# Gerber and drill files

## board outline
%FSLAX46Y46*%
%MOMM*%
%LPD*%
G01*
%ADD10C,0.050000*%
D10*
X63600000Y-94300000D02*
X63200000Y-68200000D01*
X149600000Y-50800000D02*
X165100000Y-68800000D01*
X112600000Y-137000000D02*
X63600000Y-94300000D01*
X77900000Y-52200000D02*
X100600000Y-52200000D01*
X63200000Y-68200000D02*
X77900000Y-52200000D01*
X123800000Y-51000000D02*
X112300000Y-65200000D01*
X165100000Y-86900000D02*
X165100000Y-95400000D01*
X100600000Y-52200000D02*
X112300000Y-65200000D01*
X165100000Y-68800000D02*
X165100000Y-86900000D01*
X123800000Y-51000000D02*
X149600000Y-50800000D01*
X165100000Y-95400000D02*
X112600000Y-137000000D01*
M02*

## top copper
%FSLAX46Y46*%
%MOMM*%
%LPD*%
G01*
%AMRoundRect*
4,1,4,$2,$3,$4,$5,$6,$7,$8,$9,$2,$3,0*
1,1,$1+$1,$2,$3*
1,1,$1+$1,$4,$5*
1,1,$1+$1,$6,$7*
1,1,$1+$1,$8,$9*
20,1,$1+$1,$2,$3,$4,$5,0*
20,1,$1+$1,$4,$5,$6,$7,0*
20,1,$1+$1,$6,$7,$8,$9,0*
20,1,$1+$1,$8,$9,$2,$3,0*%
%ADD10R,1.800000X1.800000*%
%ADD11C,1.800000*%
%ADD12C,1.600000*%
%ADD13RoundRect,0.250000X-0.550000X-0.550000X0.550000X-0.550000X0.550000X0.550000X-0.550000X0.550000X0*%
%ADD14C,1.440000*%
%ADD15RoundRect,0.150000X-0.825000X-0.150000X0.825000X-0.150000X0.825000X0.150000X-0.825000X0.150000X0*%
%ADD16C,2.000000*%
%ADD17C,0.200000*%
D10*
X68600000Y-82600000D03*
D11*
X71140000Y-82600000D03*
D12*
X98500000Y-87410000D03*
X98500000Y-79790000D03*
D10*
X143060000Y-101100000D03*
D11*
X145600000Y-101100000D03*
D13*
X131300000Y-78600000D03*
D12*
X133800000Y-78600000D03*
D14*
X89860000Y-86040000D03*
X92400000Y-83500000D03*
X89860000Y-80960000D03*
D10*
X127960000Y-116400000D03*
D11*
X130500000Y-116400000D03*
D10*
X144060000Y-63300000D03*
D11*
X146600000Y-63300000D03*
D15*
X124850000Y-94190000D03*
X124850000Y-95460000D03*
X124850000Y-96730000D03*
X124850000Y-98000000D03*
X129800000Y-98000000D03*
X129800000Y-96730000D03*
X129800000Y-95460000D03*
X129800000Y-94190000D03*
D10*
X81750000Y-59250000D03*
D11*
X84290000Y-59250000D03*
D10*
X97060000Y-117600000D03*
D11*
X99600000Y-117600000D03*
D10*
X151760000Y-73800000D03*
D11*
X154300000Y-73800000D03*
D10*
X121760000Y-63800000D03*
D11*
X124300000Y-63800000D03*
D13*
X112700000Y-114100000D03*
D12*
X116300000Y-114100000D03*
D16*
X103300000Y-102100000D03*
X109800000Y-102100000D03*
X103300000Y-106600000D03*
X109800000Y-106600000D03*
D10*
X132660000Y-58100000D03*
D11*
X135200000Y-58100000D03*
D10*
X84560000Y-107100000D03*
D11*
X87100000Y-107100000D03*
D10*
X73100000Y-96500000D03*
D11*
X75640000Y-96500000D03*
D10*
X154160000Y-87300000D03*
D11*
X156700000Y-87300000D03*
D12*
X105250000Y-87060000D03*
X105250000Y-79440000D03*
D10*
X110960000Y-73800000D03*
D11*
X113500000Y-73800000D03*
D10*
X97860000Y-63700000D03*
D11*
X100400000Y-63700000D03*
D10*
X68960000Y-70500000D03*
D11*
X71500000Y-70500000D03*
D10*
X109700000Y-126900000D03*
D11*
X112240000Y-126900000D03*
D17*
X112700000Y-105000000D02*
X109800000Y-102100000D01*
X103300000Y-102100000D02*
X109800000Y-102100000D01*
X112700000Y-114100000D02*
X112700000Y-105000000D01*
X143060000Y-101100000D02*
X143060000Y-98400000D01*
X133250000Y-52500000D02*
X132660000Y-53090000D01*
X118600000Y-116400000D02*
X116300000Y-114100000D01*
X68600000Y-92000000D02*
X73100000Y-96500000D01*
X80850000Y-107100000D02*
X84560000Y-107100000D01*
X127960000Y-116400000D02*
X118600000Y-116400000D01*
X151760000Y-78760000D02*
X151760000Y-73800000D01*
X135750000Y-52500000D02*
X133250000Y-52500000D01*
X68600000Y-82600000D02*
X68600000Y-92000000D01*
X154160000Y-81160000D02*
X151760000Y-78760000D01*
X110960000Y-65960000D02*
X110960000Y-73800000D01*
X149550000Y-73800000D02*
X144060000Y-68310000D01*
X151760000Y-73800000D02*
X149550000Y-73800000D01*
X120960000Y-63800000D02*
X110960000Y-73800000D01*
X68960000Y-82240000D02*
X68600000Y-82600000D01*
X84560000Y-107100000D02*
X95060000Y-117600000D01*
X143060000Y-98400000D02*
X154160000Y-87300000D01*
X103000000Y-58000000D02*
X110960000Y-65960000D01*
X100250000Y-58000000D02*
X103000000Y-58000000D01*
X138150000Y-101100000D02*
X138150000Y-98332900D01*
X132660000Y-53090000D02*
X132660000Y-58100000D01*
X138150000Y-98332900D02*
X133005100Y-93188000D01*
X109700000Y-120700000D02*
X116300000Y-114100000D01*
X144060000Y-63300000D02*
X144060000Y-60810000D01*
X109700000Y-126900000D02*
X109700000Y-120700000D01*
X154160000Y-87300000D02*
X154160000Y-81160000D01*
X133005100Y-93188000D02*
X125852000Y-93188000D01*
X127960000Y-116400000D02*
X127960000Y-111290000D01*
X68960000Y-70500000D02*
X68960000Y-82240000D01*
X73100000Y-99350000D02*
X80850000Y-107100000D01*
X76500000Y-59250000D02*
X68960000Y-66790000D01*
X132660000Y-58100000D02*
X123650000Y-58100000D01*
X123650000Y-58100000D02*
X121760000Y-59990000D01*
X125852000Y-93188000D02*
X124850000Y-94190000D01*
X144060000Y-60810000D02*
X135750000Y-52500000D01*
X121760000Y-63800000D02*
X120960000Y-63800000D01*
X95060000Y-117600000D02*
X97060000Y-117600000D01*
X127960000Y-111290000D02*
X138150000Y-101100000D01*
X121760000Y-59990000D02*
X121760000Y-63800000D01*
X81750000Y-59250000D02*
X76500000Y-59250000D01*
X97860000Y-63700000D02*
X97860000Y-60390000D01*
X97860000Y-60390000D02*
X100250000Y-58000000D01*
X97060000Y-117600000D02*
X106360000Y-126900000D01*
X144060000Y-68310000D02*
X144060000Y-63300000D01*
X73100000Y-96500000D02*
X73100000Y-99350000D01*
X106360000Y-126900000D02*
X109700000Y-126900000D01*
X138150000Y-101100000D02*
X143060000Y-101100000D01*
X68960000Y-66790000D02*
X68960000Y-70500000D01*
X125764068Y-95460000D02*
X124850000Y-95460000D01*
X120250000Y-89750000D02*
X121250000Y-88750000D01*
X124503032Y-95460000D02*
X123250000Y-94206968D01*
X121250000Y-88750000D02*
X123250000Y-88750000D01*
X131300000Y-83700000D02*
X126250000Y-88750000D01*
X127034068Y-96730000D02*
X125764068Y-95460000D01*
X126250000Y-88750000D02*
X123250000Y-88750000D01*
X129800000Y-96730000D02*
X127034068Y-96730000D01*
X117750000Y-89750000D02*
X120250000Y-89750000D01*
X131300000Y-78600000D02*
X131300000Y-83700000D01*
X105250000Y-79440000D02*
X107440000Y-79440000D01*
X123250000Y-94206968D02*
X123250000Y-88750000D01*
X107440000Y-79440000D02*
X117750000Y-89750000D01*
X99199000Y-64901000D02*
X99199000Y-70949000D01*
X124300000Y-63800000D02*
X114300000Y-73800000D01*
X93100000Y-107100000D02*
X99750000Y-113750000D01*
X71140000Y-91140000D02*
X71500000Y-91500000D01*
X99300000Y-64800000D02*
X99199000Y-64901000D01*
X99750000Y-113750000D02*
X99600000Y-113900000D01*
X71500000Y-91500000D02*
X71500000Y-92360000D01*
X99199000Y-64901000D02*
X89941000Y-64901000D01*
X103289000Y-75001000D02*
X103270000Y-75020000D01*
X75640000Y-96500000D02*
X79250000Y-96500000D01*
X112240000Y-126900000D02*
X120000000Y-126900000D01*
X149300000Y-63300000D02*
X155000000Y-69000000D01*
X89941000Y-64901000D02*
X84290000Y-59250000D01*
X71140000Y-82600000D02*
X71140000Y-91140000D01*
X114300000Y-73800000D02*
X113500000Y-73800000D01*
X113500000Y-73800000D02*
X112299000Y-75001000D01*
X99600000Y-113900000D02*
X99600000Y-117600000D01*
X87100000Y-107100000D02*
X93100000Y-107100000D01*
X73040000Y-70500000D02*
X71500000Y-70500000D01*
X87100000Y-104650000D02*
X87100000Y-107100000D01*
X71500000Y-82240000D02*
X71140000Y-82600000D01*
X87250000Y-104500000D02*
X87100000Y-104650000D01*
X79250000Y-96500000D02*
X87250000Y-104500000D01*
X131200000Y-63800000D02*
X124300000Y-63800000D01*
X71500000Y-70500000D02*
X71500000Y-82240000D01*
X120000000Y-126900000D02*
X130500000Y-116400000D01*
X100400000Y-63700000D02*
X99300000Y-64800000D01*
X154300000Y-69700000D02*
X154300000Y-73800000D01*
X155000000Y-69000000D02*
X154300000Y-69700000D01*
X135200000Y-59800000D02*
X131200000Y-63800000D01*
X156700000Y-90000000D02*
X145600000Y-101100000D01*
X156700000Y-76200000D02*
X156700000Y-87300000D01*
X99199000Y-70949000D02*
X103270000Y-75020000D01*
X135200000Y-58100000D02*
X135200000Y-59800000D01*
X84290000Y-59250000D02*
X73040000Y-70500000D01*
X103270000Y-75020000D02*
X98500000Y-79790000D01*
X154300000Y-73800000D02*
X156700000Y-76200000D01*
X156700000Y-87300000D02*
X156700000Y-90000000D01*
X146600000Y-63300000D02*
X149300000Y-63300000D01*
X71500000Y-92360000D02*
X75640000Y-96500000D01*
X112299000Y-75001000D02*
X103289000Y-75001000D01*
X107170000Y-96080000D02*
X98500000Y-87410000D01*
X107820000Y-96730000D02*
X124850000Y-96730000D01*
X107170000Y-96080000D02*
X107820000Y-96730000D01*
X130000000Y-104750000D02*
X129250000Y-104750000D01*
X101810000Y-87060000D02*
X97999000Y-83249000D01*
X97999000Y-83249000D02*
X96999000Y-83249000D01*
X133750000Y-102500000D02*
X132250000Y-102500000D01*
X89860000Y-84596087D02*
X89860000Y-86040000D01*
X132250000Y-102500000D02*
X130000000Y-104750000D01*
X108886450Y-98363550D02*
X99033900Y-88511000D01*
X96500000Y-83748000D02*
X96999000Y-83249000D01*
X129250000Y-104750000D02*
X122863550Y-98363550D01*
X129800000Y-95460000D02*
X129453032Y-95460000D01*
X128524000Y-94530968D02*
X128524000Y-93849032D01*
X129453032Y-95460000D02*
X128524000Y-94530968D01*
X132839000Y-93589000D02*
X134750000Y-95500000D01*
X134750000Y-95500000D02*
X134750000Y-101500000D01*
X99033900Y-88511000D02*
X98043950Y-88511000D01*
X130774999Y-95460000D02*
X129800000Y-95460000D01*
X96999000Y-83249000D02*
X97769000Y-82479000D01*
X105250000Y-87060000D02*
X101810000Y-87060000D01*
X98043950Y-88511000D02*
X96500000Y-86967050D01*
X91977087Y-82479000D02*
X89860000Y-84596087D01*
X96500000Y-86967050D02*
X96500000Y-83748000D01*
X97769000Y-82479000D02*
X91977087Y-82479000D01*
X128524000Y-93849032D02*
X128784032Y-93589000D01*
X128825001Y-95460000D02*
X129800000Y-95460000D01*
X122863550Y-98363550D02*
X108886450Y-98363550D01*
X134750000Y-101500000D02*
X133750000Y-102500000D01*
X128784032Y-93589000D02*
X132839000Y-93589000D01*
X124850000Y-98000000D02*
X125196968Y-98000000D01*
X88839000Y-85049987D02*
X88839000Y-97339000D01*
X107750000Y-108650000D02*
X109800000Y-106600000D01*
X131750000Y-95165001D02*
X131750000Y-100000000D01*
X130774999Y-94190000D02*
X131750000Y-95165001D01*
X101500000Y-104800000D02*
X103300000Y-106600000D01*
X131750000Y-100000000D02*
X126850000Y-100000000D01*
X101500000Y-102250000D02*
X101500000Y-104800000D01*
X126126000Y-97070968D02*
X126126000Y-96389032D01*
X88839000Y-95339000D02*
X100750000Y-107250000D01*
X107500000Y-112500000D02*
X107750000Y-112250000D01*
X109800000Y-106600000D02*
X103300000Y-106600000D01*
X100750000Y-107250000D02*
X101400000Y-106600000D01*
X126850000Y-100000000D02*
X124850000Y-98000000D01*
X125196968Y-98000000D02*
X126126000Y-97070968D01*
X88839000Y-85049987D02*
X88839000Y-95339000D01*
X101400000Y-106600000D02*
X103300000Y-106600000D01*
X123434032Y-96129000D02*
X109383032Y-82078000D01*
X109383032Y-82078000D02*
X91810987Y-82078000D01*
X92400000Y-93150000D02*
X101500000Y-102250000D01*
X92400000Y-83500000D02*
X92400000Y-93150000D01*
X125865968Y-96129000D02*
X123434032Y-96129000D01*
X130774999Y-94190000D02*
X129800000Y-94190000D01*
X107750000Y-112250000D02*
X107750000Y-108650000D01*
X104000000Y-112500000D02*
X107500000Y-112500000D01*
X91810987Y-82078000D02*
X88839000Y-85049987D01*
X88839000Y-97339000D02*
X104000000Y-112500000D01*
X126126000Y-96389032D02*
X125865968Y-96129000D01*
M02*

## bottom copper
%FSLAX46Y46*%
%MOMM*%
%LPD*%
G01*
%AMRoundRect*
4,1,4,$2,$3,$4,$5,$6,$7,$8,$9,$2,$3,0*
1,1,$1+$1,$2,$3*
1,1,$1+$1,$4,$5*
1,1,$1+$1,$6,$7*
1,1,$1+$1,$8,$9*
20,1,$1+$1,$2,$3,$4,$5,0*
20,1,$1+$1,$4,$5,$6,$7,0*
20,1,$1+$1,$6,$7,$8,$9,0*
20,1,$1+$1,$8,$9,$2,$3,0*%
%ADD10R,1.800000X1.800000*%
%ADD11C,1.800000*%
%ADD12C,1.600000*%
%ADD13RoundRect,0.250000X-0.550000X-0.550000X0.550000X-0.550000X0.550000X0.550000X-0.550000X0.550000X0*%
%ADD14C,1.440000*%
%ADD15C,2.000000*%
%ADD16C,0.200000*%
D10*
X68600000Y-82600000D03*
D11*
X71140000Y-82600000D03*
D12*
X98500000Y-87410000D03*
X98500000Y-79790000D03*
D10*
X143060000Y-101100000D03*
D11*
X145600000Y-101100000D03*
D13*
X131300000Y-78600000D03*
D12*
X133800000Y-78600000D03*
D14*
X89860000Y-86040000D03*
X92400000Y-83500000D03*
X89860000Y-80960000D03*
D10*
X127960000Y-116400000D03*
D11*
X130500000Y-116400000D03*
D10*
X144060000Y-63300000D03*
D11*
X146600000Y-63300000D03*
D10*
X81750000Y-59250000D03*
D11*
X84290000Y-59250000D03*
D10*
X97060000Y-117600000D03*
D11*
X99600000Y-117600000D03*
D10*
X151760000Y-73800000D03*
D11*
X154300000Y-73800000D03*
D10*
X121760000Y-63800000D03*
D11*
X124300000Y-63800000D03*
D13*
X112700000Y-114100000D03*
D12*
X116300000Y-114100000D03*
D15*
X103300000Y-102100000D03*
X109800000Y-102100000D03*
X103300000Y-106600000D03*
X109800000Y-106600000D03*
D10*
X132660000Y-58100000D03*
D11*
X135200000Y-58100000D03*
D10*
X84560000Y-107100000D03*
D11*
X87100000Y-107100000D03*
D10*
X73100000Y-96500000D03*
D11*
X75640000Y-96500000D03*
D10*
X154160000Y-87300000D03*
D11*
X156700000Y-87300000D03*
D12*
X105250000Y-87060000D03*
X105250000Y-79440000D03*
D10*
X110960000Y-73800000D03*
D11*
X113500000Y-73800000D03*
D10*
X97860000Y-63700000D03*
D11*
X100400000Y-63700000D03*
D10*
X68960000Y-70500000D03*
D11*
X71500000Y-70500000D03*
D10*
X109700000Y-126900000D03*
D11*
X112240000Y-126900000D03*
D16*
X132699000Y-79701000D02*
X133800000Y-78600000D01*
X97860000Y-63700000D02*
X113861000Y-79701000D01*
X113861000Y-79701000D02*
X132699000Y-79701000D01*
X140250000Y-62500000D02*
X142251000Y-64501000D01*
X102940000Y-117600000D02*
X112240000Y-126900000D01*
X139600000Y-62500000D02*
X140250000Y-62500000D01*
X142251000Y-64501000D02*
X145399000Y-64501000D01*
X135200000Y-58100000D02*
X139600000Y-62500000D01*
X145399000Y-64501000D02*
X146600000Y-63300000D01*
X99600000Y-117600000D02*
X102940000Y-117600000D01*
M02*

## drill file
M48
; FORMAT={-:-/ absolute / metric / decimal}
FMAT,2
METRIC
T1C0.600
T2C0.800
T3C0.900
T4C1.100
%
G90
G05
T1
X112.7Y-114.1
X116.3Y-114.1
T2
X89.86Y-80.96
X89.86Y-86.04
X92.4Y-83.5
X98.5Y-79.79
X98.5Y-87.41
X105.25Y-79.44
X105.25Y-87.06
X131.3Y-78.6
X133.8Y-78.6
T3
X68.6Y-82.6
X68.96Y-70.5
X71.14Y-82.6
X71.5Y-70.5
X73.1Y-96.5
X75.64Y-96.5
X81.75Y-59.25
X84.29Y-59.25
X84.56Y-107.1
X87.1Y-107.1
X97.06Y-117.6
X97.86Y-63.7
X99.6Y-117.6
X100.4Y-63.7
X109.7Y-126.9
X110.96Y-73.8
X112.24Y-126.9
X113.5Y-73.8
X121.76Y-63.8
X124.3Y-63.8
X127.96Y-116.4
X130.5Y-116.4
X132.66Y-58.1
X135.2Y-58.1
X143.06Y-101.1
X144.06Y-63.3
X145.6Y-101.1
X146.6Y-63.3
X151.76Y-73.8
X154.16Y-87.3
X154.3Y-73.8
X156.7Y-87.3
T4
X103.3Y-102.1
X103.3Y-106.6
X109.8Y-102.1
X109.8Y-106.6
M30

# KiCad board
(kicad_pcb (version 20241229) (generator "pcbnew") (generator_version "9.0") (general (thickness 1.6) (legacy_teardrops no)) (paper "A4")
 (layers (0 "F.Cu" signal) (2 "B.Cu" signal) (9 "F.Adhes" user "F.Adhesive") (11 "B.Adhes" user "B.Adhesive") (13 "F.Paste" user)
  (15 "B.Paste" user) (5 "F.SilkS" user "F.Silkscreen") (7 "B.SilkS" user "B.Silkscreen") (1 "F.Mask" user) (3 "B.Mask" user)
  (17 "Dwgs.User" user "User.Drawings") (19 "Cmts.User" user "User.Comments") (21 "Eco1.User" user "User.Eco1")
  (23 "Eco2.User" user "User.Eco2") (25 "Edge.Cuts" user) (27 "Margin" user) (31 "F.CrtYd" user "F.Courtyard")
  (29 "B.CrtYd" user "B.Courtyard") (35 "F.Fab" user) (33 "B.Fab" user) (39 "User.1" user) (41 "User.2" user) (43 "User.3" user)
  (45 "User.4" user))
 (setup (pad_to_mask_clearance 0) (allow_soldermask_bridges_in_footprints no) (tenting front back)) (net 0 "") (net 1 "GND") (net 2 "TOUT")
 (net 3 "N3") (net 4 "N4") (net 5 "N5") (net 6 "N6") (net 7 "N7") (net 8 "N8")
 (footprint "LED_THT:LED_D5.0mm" (layer "F.Cu") (at 68.6 82.6)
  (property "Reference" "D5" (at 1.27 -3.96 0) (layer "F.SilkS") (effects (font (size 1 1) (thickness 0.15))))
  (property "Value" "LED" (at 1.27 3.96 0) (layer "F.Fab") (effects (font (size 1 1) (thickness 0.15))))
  (pad "1" thru_hole rect (at 0 0) (size 1.8 1.8) (drill 0.9) (layers "*.Cu" "*.Mask") (remove_unused_layers no) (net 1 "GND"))
  (pad "2" thru_hole circle (at 2.54 0) (size 1.8 1.8) (drill 0.9) (layers "*.Cu" "*.Mask") (remove_unused_layers no) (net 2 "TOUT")))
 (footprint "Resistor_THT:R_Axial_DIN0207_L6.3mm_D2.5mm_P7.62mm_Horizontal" (layer "F.Cu") (at 98.5 87.41 90)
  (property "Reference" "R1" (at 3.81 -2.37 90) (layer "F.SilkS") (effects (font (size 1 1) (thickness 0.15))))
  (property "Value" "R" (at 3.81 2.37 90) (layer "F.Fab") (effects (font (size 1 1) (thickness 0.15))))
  (pad "1" thru_hole circle (at 0 0 90) (size 1.6 1.6) (drill 0.8) (layers "*.Cu" "*.Mask") (remove_unused_layers no) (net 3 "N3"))
  (pad "2" thru_hole circle (at 7.62 0 90) (size 1.6 1.6) (drill 0.8) (layers "*.Cu" "*.Mask") (remove_unused_layers no) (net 2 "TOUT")))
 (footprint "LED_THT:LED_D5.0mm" (layer "F.Cu") (at 143.06 101.1)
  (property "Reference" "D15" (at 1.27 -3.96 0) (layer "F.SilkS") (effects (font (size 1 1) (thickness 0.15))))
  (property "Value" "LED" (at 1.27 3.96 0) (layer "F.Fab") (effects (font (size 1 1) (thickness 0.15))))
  (pad "1" thru_hole rect (at 0 0) (size 1.8 1.8) (drill 0.9) (layers "*.Cu" "*.Mask") (remove_unused_layers no) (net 1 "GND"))
  (pad "2" thru_hole circle (at 2.54 0) (size 1.8 1.8) (drill 0.9) (layers "*.Cu" "*.Mask") (remove_unused_layers no) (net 2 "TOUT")))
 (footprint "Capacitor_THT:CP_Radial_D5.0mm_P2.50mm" (layer "F.Cu") (at 131.3 78.6)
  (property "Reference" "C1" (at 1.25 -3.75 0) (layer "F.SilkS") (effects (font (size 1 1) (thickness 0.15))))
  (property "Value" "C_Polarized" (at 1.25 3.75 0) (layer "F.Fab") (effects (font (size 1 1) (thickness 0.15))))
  (pad "1" thru_hole roundrect (at 0 0) (size 1.6 1.6) (drill 0.8) (layers "*.Cu" "*.Mask") (remove_unused_layers no)
   (roundrect_rratio 0.15625) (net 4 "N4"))
  (pad "2" thru_hole circle (at 2.5 0) (size 1.6 1.6) (drill 0.8) (layers "*.Cu" "*.Mask") (remove_unused_layers no) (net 1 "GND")))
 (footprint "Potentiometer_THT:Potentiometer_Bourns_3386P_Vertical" (layer "F.Cu") (at 89.86 86.04)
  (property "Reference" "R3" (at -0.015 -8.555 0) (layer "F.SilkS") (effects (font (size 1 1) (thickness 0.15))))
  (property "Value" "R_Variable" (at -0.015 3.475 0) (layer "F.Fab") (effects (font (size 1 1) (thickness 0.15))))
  (pad "1" thru_hole circle (at 0 0) (size 1.44 1.44) (drill 0.8) (layers "*.Cu" "*.Mask") (remove_unused_layers no) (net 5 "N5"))
  (pad "2" thru_hole circle (at 2.54 -2.54) (size 1.44 1.44) (drill 0.8) (layers "*.Cu" "*.Mask") (remove_unused_layers no) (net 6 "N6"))
  (pad "3" thru_hole circle (at 0 -5.08) (size 1.44 1.44) (drill 0.8) (layers "*.Cu" "*.Mask") (remove_unused_layers no)))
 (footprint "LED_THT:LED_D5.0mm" (layer "F.Cu") (at 127.96 116.4)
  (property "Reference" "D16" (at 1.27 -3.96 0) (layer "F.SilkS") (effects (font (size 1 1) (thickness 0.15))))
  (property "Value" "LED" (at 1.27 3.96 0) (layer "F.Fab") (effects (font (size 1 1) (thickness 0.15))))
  (pad "1" thru_hole rect (at 0 0) (size 1.8 1.8) (drill 0.9) (layers "*.Cu" "*.Mask") (remove_unused_layers no) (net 1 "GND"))
  (pad "2" thru_hole circle (at 2.54 0) (size 1.8 1.8) (drill 0.9) (layers "*.Cu" "*.Mask") (remove_unused_layers no) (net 2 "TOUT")))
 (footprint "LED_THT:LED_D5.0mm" (layer "F.Cu") (at 144.06 63.3)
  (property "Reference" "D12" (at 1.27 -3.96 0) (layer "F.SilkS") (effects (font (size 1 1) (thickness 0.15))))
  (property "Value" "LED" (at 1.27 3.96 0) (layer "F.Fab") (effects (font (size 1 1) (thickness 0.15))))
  (pad "1" thru_hole rect (at 0 0) (size 1.8 1.8) (drill 0.9) (layers "*.Cu" "*.Mask") (remove_unused_layers no) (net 1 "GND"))
  (pad "2" thru_hole circle (at 2.54 0) (size 1.8 1.8) (drill 0.9) (layers "*.Cu" "*.Mask") (remove_unused_layers no) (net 2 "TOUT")))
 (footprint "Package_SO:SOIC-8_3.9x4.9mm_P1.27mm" (layer "F.Cu") (at 127.325 96.095)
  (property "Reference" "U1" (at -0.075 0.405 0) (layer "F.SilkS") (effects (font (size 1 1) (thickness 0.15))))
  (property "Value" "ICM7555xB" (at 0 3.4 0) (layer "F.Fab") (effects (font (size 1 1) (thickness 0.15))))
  (pad "1" smd roundrect (at -2.475 -1.905) (size 1.95 0.6) (layers "F.Cu" "F.Mask" "F.Paste") (roundrect_rratio 0.25) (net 1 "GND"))
  (pad "2" smd roundrect (at -2.475 -0.635) (size 1.95 0.6) (layers "F.Cu" "F.Mask" "F.Paste") (roundrect_rratio 0.25) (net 4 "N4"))
  (pad "3" smd roundrect (at -2.475 0.635) (size 1.95 0.6) (layers "F.Cu" "F.Mask" "F.Paste") (roundrect_rratio 0.25) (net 3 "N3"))
  (pad "4" smd roundrect (at -2.475 1.905) (size 1.95 0.6) (layers "F.Cu" "F.Mask" "F.Paste") (roundrect_rratio 0.25) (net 6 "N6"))
  (pad "5" smd roundrect (at 2.475 1.905) (size 1.95 0.6) (layers "F.Cu" "F.Mask" "F.Paste") (roundrect_rratio 0.25) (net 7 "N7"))
  (pad "6" smd roundrect (at 2.475 0.635) (size 1.95 0.6) (layers "F.Cu" "F.Mask" "F.Paste") (roundrect_rratio 0.25) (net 4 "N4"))
  (pad "7" smd roundrect (at 2.475 -0.635) (size 1.95 0.6) (layers "F.Cu" "F.Mask" "F.Paste") (roundrect_rratio 0.25) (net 5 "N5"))
  (pad "8" smd roundrect (at 2.475 -1.905) (size 1.95 0.6) (layers "F.Cu" "F.Mask" "F.Paste") (roundrect_rratio 0.25) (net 6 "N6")))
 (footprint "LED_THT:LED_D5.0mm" (layer "F.Cu") (at 81.75 59.25)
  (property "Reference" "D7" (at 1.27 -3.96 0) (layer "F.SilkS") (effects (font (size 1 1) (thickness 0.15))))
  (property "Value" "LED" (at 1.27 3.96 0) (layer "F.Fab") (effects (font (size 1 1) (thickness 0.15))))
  (pad "1" thru_hole rect (at 0 0) (size 1.8 1.8) (drill 0.9) (layers "*.Cu" "*.Mask") (remove_unused_layers no) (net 1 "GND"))
  (pad "2" thru_hole circle (at 2.54 0) (size 1.8 1.8) (drill 0.9) (layers "*.Cu" "*.Mask") (remove_unused_layers no) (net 2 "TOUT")))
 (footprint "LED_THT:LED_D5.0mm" (layer "F.Cu") (at 97.06 117.6)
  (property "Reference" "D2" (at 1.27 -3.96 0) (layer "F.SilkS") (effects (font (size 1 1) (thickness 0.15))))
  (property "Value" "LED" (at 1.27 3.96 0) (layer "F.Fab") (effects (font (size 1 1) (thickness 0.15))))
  (pad "1" thru_hole rect (at 0 0) (size 1.8 1.8) (drill 0.9) (layers "*.Cu" "*.Mask") (remove_unused_layers no) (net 1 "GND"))
  (pad "2" thru_hole circle (at 2.54 0) (size 1.8 1.8) (drill 0.9) (layers "*.Cu" "*.Mask") (remove_unused_layers no) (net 2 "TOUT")))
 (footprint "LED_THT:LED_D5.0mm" (layer "F.Cu") (at 151.76 73.8)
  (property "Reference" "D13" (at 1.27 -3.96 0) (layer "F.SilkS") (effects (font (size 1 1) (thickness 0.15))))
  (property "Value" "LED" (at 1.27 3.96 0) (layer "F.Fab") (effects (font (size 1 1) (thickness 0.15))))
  (pad "1" thru_hole rect (at 0 0) (size 1.8 1.8) (drill 0.9) (layers "*.Cu" "*.Mask") (remove_unused_layers no) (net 1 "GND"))
  (pad "2" thru_hole circle (at 2.54 0) (size 1.8 1.8) (drill 0.9) (layers "*.Cu" "*.Mask") (remove_unused_layers no) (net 2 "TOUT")))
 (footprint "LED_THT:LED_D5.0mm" (layer "F.Cu") (at 121.76 63.8)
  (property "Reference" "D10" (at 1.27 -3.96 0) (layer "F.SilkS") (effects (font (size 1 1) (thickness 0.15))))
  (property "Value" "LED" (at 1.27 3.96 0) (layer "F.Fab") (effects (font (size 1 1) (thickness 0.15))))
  (pad "1" thru_hole rect (at 0 0) (size 1.8 1.8) (drill 0.9) (layers "*.Cu" "*.Mask") (remove_unused_layers no) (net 1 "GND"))
  (pad "2" thru_hole circle (at 2.54 0) (size 1.8 1.8) (drill 0.9) (layers "*.Cu" "*.Mask") (remove_unused_layers no) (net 2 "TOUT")))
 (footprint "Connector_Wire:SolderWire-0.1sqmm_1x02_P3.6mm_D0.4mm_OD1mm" (layer "F.Cu") (at 112.7 114.1)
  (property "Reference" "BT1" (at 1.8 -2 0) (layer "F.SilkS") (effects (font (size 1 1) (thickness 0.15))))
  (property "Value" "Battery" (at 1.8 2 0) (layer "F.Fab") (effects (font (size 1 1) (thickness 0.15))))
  (pad "1" thru_hole roundrect (at 0 0) (size 1.6 1.6) (drill 0.6) (layers "*.Cu" "*.Mask") (remove_unused_layers no)
   (roundrect_rratio 0.15625) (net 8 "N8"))
  (pad "2" thru_hole circle (at 3.6 0) (size 1.6 1.6) (drill 0.6) (layers "*.Cu" "*.Mask") (remove_unused_layers no) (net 1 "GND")))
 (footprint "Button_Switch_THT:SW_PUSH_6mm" (layer "F.Cu") (at 103.3 102.1)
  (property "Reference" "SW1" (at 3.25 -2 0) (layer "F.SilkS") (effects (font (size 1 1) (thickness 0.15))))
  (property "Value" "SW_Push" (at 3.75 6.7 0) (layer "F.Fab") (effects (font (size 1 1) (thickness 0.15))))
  (pad "1" thru_hole circle (at 0 0 90) (size 2 2) (drill 1.1) (layers "*.Cu" "*.Mask") (remove_unused_layers no) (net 8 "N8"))
  (pad "1" thru_hole circle (at 6.5 0 90) (size 2 2) (drill 1.1) (layers "*.Cu" "*.Mask") (remove_unused_layers no) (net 8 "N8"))
  (pad "2" thru_hole circle (at 0 4.5 90) (size 2 2) (drill 1.1) (layers "*.Cu" "*.Mask") (remove_unused_layers no) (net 6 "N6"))
  (pad "2" thru_hole circle (at 6.5 4.5 90) (size 2 2) (drill 1.1) (layers "*.Cu" "*.Mask") (remove_unused_layers no) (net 6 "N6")))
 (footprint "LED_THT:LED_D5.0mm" (layer "F.Cu") (at 132.66 58.1)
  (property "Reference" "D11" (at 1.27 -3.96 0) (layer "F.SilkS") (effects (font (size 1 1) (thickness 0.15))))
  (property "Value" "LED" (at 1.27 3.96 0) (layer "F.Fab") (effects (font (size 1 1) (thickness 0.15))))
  (pad "1" thru_hole rect (at 0 0) (size 1.8 1.8) (drill 0.9) (layers "*.Cu" "*.Mask") (remove_unused_layers no) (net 1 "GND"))
  (pad "2" thru_hole circle (at 2.54 0) (size 1.8 1.8) (drill 0.9) (layers "*.Cu" "*.Mask") (remove_unused_layers no) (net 2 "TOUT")))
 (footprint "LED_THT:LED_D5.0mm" (layer "F.Cu") (at 84.56 107.1)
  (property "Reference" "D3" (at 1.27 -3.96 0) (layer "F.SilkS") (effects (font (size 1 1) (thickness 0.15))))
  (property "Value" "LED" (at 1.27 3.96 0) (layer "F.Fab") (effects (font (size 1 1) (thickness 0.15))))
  (pad "1" thru_hole rect (at 0 0) (size 1.8 1.8) (drill 0.9) (layers "*.Cu" "*.Mask") (remove_unused_layers no) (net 1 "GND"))
  (pad "2" thru_hole circle (at 2.54 0) (size 1.8 1.8) (drill 0.9) (layers "*.Cu" "*.Mask") (remove_unused_layers no) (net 2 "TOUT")))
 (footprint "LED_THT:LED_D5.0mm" (layer "F.Cu") (at 73.1 96.5)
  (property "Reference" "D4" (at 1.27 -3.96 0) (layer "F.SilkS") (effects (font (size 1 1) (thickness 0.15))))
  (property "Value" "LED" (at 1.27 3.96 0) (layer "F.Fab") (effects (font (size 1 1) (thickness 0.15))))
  (pad "1" thru_hole rect (at 0 0) (size 1.8 1.8) (drill 0.9) (layers "*.Cu" "*.Mask") (remove_unused_layers no) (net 1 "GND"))
  (pad "2" thru_hole circle (at 2.54 0) (size 1.8 1.8) (drill 0.9) (layers "*.Cu" "*.Mask") (remove_unused_layers no) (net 2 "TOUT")))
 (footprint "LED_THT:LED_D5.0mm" (layer "F.Cu") (at 154.16 87.3)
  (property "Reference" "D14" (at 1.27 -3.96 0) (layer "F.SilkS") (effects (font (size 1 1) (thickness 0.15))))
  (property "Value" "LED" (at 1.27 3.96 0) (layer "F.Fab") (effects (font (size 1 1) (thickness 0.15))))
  (pad "1" thru_hole rect (at 0 0) (size 1.8 1.8) (drill 0.9) (layers "*.Cu" "*.Mask") (remove_unused_layers no) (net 1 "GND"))
  (pad "2" thru_hole circle (at 2.54 0) (size 1.8 1.8) (drill 0.9) (layers "*.Cu" "*.Mask") (remove_unused_layers no) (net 2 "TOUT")))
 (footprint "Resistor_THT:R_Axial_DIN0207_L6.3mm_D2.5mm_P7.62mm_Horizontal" (layer "F.Cu") (at 105.25 87.06 90)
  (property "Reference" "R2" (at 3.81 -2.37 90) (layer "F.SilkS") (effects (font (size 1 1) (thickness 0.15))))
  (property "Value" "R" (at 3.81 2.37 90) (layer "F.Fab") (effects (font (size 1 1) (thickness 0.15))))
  (pad "1" thru_hole circle (at 0 0 90) (size 1.6 1.6) (drill 0.8) (layers "*.Cu" "*.Mask") (remove_unused_layers no) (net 5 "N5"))
  (pad "2" thru_hole circle (at 7.62 0 90) (size 1.6 1.6) (drill 0.8) (layers "*.Cu" "*.Mask") (remove_unused_layers no) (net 4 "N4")))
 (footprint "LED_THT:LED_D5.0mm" (layer "F.Cu") (at 110.96 73.8)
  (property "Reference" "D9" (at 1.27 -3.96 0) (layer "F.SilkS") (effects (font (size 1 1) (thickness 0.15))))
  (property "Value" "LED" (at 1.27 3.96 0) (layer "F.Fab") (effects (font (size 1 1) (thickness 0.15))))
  (pad "1" thru_hole rect (at 0 0) (size 1.8 1.8) (drill 0.9) (layers "*.Cu" "*.Mask") (remove_unused_layers no) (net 1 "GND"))
  (pad "2" thru_hole circle (at 2.54 0) (size 1.8 1.8) (drill 0.9) (layers "*.Cu" "*.Mask") (remove_unused_layers no) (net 2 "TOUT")))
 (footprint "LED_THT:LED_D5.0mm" (layer "F.Cu") (at 97.86 63.7)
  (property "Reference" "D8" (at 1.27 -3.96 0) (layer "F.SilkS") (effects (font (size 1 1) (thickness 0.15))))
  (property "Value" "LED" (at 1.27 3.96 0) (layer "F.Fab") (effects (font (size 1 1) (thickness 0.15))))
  (pad "1" thru_hole rect (at 0 0) (size 1.8 1.8) (drill 0.9) (layers "*.Cu" "*.Mask") (remove_unused_layers no) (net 1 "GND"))
  (pad "2" thru_hole circle (at 2.54 0) (size 1.8 1.8) (drill 0.9) (layers "*.Cu" "*.Mask") (remove_unused_layers no) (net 2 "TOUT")))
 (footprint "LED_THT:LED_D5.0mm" (layer "F.Cu") (at 68.96 70.5)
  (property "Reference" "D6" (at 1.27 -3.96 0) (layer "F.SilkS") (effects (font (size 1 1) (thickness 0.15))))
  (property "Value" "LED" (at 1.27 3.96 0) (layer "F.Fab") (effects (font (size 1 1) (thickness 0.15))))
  (pad "1" thru_hole rect (at 0 0) (size 1.8 1.8) (drill 0.9) (layers "*.Cu" "*.Mask") (remove_unused_layers no) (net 1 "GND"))
  (pad "2" thru_hole circle (at 2.54 0) (size 1.8 1.8) (drill 0.9) (layers "*.Cu" "*.Mask") (remove_unused_layers no) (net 2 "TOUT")))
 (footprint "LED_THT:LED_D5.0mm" (layer "F.Cu") (at 109.7 126.9)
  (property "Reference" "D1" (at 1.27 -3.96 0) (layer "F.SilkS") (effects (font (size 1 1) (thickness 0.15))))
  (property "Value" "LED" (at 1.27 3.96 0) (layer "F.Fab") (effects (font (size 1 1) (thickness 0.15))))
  (pad "1" thru_hole rect (at 0 0) (size 1.8 1.8) (drill 0.9) (layers "*.Cu" "*.Mask") (remove_unused_layers no) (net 1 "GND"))
  (pad "2" thru_hole circle (at 2.54 0) (size 1.8 1.8) (drill 0.9) (layers "*.Cu" "*.Mask") (remove_unused_layers no) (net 2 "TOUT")))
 (gr_line (start 63.6 94.3) (end 63.2 68.2) (stroke (width 0.05) (type default)) (layer "Edge.Cuts"))
 (gr_line (start 149.6 50.8) (end 165.1 68.8) (stroke (width 0.05) (type default)) (layer "Edge.Cuts"))
 (gr_line (start 112.6 137) (end 63.6 94.3) (stroke (width 0.05) (type default)) (layer "Edge.Cuts"))
 (gr_line (start 77.9 52.2) (end 100.6 52.2) (stroke (width 0.05) (type default)) (layer "Edge.Cuts"))
 (gr_line (start 63.2 68.2) (end 77.9 52.2) (stroke (width 0.05) (type default)) (layer "Edge.Cuts"))
 (gr_line (start 123.8 51) (end 112.3 65.2) (stroke (width 0.05) (type default)) (layer "Edge.Cuts"))
 (gr_line (start 165.1 86.9) (end 165.1 95.4) (stroke (width 0.05) (type default)) (layer "Edge.Cuts"))
 (gr_line (start 100.6 52.2) (end 112.3 65.2) (stroke (width 0.05) (type default)) (layer "Edge.Cuts"))
 (gr_line (start 165.1 68.8) (end 165.1 86.9) (stroke (width 0.05) (type default)) (layer "Edge.Cuts"))
 (gr_line (start 123.8 51) (end 149.6 50.8) (stroke (width 0.05) (type default)) (layer "Edge.Cuts"))
 (gr_line (start 165.1 95.4) (end 112.6 137) (stroke (width 0.05) (type default)) (layer "Edge.Cuts"))
 (segment (start 112.7 105) (end 109.8 102.1) (width 0.2) (layer "F.Cu") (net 8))
 (segment (start 103.3 102.1) (end 109.8 102.1) (width 0.2) (layer "F.Cu") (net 8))
 (segment (start 112.7 114.1) (end 112.7 105) (width 0.2) (layer "F.Cu") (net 8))
 (segment (start 143.06 101.1) (end 143.06 98.4) (width 0.2) (layer "F.Cu") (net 1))
 (segment (start 133.25 52.5) (end 132.66 53.09) (width 0.2) (layer "F.Cu") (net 1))
 (segment (start 118.6 116.4) (end 116.3 114.1) (width 0.2) (layer "F.Cu") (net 1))
 (segment (start 68.6 92) (end 73.1 96.5) (width 0.2) (layer "F.Cu") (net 1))
 (segment (start 80.85 107.1) (end 84.56 107.1) (width 0.2) (layer "F.Cu") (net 1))
 (segment (start 127.96 116.4) (end 118.6 116.4) (width 0.2) (layer "F.Cu") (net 1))
 (segment (start 151.76 78.76) (end 151.76 73.8) (width 0.2) (layer "F.Cu") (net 1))
 (segment (start 135.75 52.5) (end 133.25 52.5) (width 0.2) (layer "F.Cu") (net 1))
 (segment (start 68.6 82.6) (end 68.6 92) (width 0.2) (layer "F.Cu") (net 1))
 (segment (start 154.16 81.16) (end 151.76 78.76) (width 0.2) (layer "F.Cu") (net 1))
 (segment (start 110.96 65.96) (end 110.96 73.8) (width 0.2) (layer "F.Cu") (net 1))
 (segment (start 149.55 73.8) (end 144.06 68.31) (width 0.2) (layer "F.Cu") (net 1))
 (segment (start 151.76 73.8) (end 149.55 73.8) (width 0.2) (layer "F.Cu") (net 1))
 (segment (start 120.96 63.8) (end 110.96 73.8) (width 0.2) (layer "F.Cu") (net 1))
 (segment (start 68.96 82.24) (end 68.6 82.6) (width 0.2) (layer "F.Cu") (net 1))
 (segment (start 84.56 107.1) (end 95.06 117.6) (width 0.2) (layer "F.Cu") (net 1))
 (segment (start 143.06 98.4) (end 154.16 87.3) (width 0.2) (layer "F.Cu") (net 1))
 (segment (start 103 58) (end 110.96 65.96) (width 0.2) (layer "F.Cu") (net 1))
 (segment (start 100.25 58) (end 103 58) (width 0.2) (layer "F.Cu") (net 1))
 (segment (start 138.15 101.1) (end 138.15 98.3329) (width 0.2) (layer "F.Cu") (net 1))
 (segment (start 132.66 53.09) (end 132.66 58.1) (width 0.2) (layer "F.Cu") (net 1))
 (segment (start 138.15 98.3329) (end 133.0051 93.188) (width 0.2) (layer "F.Cu") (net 1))
 (segment (start 109.7 120.7) (end 116.3 114.1) (width 0.2) (layer "F.Cu") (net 1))
 (segment (start 144.06 63.3) (end 144.06 60.81) (width 0.2) (layer "F.Cu") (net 1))
 (segment (start 109.7 126.9) (end 109.7 120.7) (width 0.2) (layer "F.Cu") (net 1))
 (segment (start 154.16 87.3) (end 154.16 81.16) (width 0.2) (layer "F.Cu") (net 1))
 (segment (start 133.0051 93.188) (end 125.852 93.188) (width 0.2) (layer "F.Cu") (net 1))
 (segment (start 127.96 116.4) (end 127.96 111.29) (width 0.2) (layer "F.Cu") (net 1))
 (segment (start 68.96 70.5) (end 68.96 82.24) (width 0.2) (layer "F.Cu") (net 1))
 (segment (start 73.1 99.35) (end 80.85 107.1) (width 0.2) (layer "F.Cu") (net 1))
 (segment (start 76.5 59.25) (end 68.96 66.79) (width 0.2) (layer "F.Cu") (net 1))
 (segment (start 132.66 58.1) (end 123.65 58.1) (width 0.2) (layer "F.Cu") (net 1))
 (segment (start 123.65 58.1) (end 121.76 59.99) (width 0.2) (layer "F.Cu") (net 1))
 (segment (start 125.852 93.188) (end 124.85 94.19) (width 0.2) (layer "F.Cu") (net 1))
 (segment (start 144.06 60.81) (end 135.75 52.5) (width 0.2) (layer "F.Cu") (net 1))
 (segment (start 121.76 63.8) (end 120.96 63.8) (width 0.2) (layer "F.Cu") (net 1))
 (segment (start 95.06 117.6) (end 97.06 117.6) (width 0.2) (layer "F.Cu") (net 1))
 (segment (start 127.96 111.29) (end 138.15 101.1) (width 0.2) (layer "F.Cu") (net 1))
 (segment (start 121.76 59.99) (end 121.76 63.8) (width 0.2) (layer "F.Cu") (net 1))
 (segment (start 81.75 59.25) (end 76.5 59.25) (width 0.2) (layer "F.Cu") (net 1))
 (segment (start 97.86 63.7) (end 97.86 60.39) (width 0.2) (layer "F.Cu") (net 1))
 (segment (start 97.86 60.39) (end 100.25 58) (width 0.2) (layer "F.Cu") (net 1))
 (segment (start 97.06 117.6) (end 106.36 126.9) (width 0.2) (layer "F.Cu") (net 1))
 (segment (start 144.06 68.31) (end 144.06 63.3) (width 0.2) (layer "F.Cu") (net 1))
 (segment (start 73.1 96.5) (end 73.1 99.35) (width 0.2) (layer "F.Cu") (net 1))
 (segment (start 106.36 126.9) (end 109.7 126.9) (width 0.2) (layer "F.Cu") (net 1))
 (segment (start 138.15 101.1) (end 143.06 101.1) (width 0.2) (layer "F.Cu") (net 1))
 (segment (start 68.96 66.79) (end 68.96 70.5) (width 0.2) (layer "F.Cu") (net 1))
 (segment (start 132.699 79.701) (end 133.8 78.6) (width 0.2) (layer "B.Cu") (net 1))
 (segment (start 97.86 63.7) (end 113.861 79.701) (width 0.2) (layer "B.Cu") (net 1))
 (segment (start 113.861 79.701) (end 132.699 79.701) (width 0.2) (layer "B.Cu") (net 1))
 (segment (start 125.764068 95.46) (end 124.85 95.46) (width 0.2) (layer "F.Cu") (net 4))
 (segment (start 120.25 89.75) (end 121.25 88.75) (width 0.2) (layer "F.Cu") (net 4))
 (segment (start 124.503032 95.46) (end 123.25 94.206968) (width 0.2) (layer "F.Cu") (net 4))
 (segment (start 121.25 88.75) (end 123.25 88.75) (width 0.2) (layer "F.Cu") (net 4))
 (segment (start 131.3 83.7) (end 126.25 88.75) (width 0.2) (layer "F.Cu") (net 4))
 (segment (start 127.034068 96.73) (end 125.764068 95.46) (width 0.2) (layer "F.Cu") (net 4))
 (segment (start 126.25 88.75) (end 123.25 88.75) (width 0.2) (layer "F.Cu") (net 4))
 (segment (start 129.8 96.73) (end 127.034068 96.73) (width 0.2) (layer "F.Cu") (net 4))
 (segment (start 117.75 89.75) (end 120.25 89.75) (width 0.2) (layer "F.Cu") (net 4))
 (segment (start 131.3 78.6) (end 131.3 83.7) (width 0.2) (layer "F.Cu") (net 4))
 (segment (start 105.25 79.44) (end 107.44 79.44) (width 0.2) (layer "F.Cu") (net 4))
 (segment (start 123.25 94.206968) (end 123.25 88.75) (width 0.2) (layer "F.Cu") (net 4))
 (segment (start 107.44 79.44) (end 117.75 89.75) (width 0.2) (layer "F.Cu") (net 4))
 (segment (start 99.199 64.901) (end 99.199 70.949) (width 0.2) (layer "F.Cu") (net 2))
 (segment (start 124.3 63.8) (end 114.3 73.8) (width 0.2) (layer "F.Cu") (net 2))
 (segment (start 93.1 107.1) (end 99.75 113.75) (width 0.2) (layer "F.Cu") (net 2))
 (segment (start 71.14 91.14) (end 71.5 91.5) (width 0.2) (layer "F.Cu") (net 2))
 (segment (start 99.3 64.8) (end 99.199 64.901) (width 0.2) (layer "F.Cu") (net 2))
 (segment (start 99.75 113.75) (end 99.6 113.9) (width 0.2) (layer "F.Cu") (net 2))
 (segment (start 71.5 91.5) (end 71.5 92.36) (width 0.2) (layer "F.Cu") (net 2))
 (segment (start 99.199 64.901) (end 89.941 64.901) (width 0.2) (layer "F.Cu") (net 2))
 (segment (start 103.289 75.001) (end 103.27 75.02) (width 0.2) (layer "F.Cu") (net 2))
 (segment (start 75.64 96.5) (end 79.25 96.5) (width 0.2) (layer "F.Cu") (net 2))
 (segment (start 112.24 126.9) (end 120 126.9) (width 0.2) (layer "F.Cu") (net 2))
 (segment (start 149.3 63.3) (end 155 69) (width 0.2) (layer "F.Cu") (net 2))
 (segment (start 89.941 64.901) (end 84.29 59.25) (width 0.2) (layer "F.Cu") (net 2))
 (segment (start 71.14 82.6) (end 71.14 91.14) (width 0.2) (layer "F.Cu") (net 2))
 (segment (start 114.3 73.8) (end 113.5 73.8) (width 0.2) (layer "F.Cu") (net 2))
 (segment (start 113.5 73.8) (end 112.299 75.001) (width 0.2) (layer "F.Cu") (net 2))
 (segment (start 99.6 113.9) (end 99.6 117.6) (width 0.2) (layer "F.Cu") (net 2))
 (segment (start 87.1 107.1) (end 93.1 107.1) (width 0.2) (layer "F.Cu") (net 2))
 (segment (start 73.04 70.5) (end 71.5 70.5) (width 0.2) (layer "F.Cu") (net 2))
 (segment (start 87.1 104.65) (end 87.1 107.1) (width 0.2) (layer "F.Cu") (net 2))
 (segment (start 71.5 82.24) (end 71.14 82.6) (width 0.2) (layer "F.Cu") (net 2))
 (segment (start 87.25 104.5) (end 87.1 104.65) (width 0.2) (layer "F.Cu") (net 2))
 (segment (start 79.25 96.5) (end 87.25 104.5) (width 0.2) (layer "F.Cu") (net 2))
 (segment (start 131.2 63.8) (end 124.3 63.8) (width 0.2) (layer "F.Cu") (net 2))
 (segment (start 71.5 70.5) (end 71.5 82.24) (width 0.2) (layer "F.Cu") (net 2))
 (segment (start 120 126.9) (end 130.5 116.4) (width 0.2) (layer "F.Cu") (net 2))
 (segment (start 100.4 63.7) (end 99.3 64.8) (width 0.2) (layer "F.Cu") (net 2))
 (segment (start 154.3 69.7) (end 154.3 73.8) (width 0.2) (layer "F.Cu") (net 2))
 (segment (start 155 69) (end 154.3 69.7) (width 0.2) (layer "F.Cu") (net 2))
 (segment (start 135.2 59.8) (end 131.2 63.8) (width 0.2) (layer "F.Cu") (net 2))
 (segment (start 156.7 90) (end 145.6 101.1) (width 0.2) (layer "F.Cu") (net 2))
 (segment (start 156.7 76.2) (end 156.7 87.3) (width 0.2) (layer "F.Cu") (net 2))
 (segment (start 99.199 70.949) (end 103.27 75.02) (width 0.2) (layer "F.Cu") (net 2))
 (segment (start 135.2 58.1) (end 135.2 59.8) (width 0.2) (layer "F.Cu") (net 2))
 (segment (start 84.29 59.25) (end 73.04 70.5) (width 0.2) (layer "F.Cu") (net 2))
 (segment (start 103.27 75.02) (end 98.5 79.79) (width 0.2) (layer "F.Cu") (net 2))
 (segment (start 154.3 73.8) (end 156.7 76.2) (width 0.2) (layer "F.Cu") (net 2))
 (segment (start 156.7 87.3) (end 156.7 90) (width 0.2) (layer "F.Cu") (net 2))
 (segment (start 146.6 63.3) (end 149.3 63.3) (width 0.2) (layer "F.Cu") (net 2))
 (segment (start 71.5 92.36) (end 75.64 96.5) (width 0.2) (layer "F.Cu") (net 2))
 (segment (start 112.299 75.001) (end 103.289 75.001) (width 0.2) (layer "F.Cu") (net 2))
 (segment (start 140.25 62.5) (end 142.251 64.501) (width 0.2) (layer "B.Cu") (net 2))
 (segment (start 102.94 117.6) (end 112.24 126.9) (width 0.2) (layer "B.Cu") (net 2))
 (segment (start 139.6 62.5) (end 140.25 62.5) (width 0.2) (layer "B.Cu") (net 2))
 (segment (start 142.251 64.501) (end 145.399 64.501) (width 0.2) (layer "B.Cu") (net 2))
 (segment (start 135.2 58.1) (end 139.6 62.5) (width 0.2) (layer "B.Cu") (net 2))
 (segment (start 145.399 64.501) (end 146.6 63.3) (width 0.2) (layer "B.Cu") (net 2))
 (segment (start 99.6 117.6) (end 102.94 117.6) (width 0.2) (layer "B.Cu") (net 2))
 (segment (start 107.17 96.08) (end 98.5 87.41) (width 0.2) (layer "F.Cu") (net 3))
 (segment (start 107.82 96.73) (end 124.85 96.73) (width 0.2) (layer "F.Cu") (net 3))
 (segment (start 107.17 96.08) (end 107.82 96.73) (width 0.2) (layer "F.Cu") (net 3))
 (segment (start 130 104.75) (end 129.25 104.75) (width 0.2) (layer "F.Cu") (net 5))
 (segment (start 101.81 87.06) (end 97.999 83.249) (width 0.2) (layer "F.Cu") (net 5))
 (segment (start 97.999 83.249) (end 96.999 83.249) (width 0.2) (layer "F.Cu") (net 5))
 (segment (start 133.75 102.5) (end 132.25 102.5) (width 0.2) (layer "F.Cu") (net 5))
 (segment (start 89.86 84.596087) (end 89.86 86.04) (width 0.2) (layer "F.Cu") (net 5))
 (segment (start 132.25 102.5) (end 130 104.75) (width 0.2) (layer "F.Cu") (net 5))
 (segment (start 108.88645 98.36355) (end 99.0339 88.511) (width 0.2) (layer "F.Cu") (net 5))
 (segment (start 96.5 83.748) (end 96.999 83.249) (width 0.2) (layer "F.Cu") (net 5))
 (segment (start 129.25 104.75) (end 122.86355 98.36355) (width 0.2) (layer "F.Cu") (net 5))
 (segment (start 129.8 95.46) (end 129.453032 95.46) (width 0.2) (layer "F.Cu") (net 5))
 (segment (start 128.524 94.530968) (end 128.524 93.849032) (width 0.2) (layer "F.Cu") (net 5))
 (segment (start 129.453032 95.46) (end 128.524 94.530968) (width 0.2) (layer "F.Cu") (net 5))
 (segment (start 132.839 93.589) (end 134.75 95.5) (width 0.2) (layer "F.Cu") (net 5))
 (segment (start 134.75 95.5) (end 134.75 101.5) (width 0.2) (layer "F.Cu") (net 5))
 (segment (start 99.0339 88.511) (end 98.04395 88.511) (width 0.2) (layer "F.Cu") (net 5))
 (segment (start 130.774999 95.46) (end 129.8 95.46) (width 0.2) (layer "F.Cu") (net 5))
 (segment (start 96.999 83.249) (end 97.769 82.479) (width 0.2) (layer "F.Cu") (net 5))
 (segment (start 105.25 87.06) (end 101.81 87.06) (width 0.2) (layer "F.Cu") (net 5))
 (segment (start 98.04395 88.511) (end 96.5 86.96705) (width 0.2) (layer "F.Cu") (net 5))
 (segment (start 91.977087 82.479) (end 89.86 84.596087) (width 0.2) (layer "F.Cu") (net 5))
 (segment (start 96.5 86.96705) (end 96.5 83.748) (width 0.2) (layer "F.Cu") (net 5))
 (segment (start 97.769 82.479) (end 91.977087 82.479) (width 0.2) (layer "F.Cu") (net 5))
 (segment (start 128.524 93.849032) (end 128.784032 93.589) (width 0.2) (layer "F.Cu") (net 5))
 (segment (start 128.825001 95.46) (end 129.8 95.46) (width 0.2) (layer "F.Cu") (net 5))
 (segment (start 122.86355 98.36355) (end 108.88645 98.36355) (width 0.2) (layer "F.Cu") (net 5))
 (segment (start 134.75 101.5) (end 133.75 102.5) (width 0.2) (layer "F.Cu") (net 5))
 (segment (start 128.784032 93.589) (end 132.839 93.589) (width 0.2) (layer "F.Cu") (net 5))
 (segment (start 124.85 98) (end 125.196968 98) (width 0.2) (layer "F.Cu") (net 6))
 (segment (start 88.839 85.049987) (end 88.839 97.339) (width 0.2) (layer "F.Cu") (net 6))
 (segment (start 107.75 108.65) (end 109.8 106.6) (width 0.2) (layer "F.Cu") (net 6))
 (segment (start 131.75 95.165001) (end 131.75 100) (width 0.2) (layer "F.Cu") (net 6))
 (segment (start 130.774999 94.19) (end 131.75 95.165001) (width 0.2) (layer "F.Cu") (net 6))
 (segment (start 101.5 104.8) (end 103.3 106.6) (width 0.2) (layer "F.Cu") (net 6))
 (segment (start 131.75 100) (end 126.85 100) (width 0.2) (layer "F.Cu") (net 6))
 (segment (start 101.5 102.25) (end 101.5 104.8) (width 0.2) (layer "F.Cu") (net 6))
 (segment (start 126.126 97.070968) (end 126.126 96.389032) (width 0.2) (layer "F.Cu") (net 6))
 (segment (start 88.839 95.339) (end 100.75 107.25) (width 0.2) (layer "F.Cu") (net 6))
 (segment (start 107.5 112.5) (end 107.75 112.25) (width 0.2) (layer "F.Cu") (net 6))
 (segment (start 109.8 106.6) (end 103.3 106.6) (width 0.2) (layer "F.Cu") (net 6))
 (segment (start 100.75 107.25) (end 101.4 106.6) (width 0.2) (layer "F.Cu") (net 6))
 (segment (start 126.85 100) (end 124.85 98) (width 0.2) (layer "F.Cu") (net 6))
 (segment (start 125.196968 98) (end 126.126 97.070968) (width 0.2) (layer "F.Cu") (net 6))
 (segment (start 88.839 85.049987) (end 88.839 95.339) (width 0.2) (layer "F.Cu") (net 6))
 (segment (start 101.4 106.6) (end 103.3 106.6) (width 0.2) (layer "F.Cu") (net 6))
 (segment (start 123.434032 96.129) (end 109.383032 82.078) (width 0.2) (layer "F.Cu") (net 6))
 (segment (start 109.383032 82.078) (end 91.810987 82.078) (width 0.2) (layer "F.Cu") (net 6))
 (segment (start 92.4 93.15) (end 101.5 102.25) (width 0.2) (layer "F.Cu") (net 6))
 (segment (start 92.4 83.5) (end 92.4 93.15) (width 0.2) (layer "F.Cu") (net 6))
 (segment (start 125.865968 96.129) (end 123.434032 96.129) (width 0.2) (layer "F.Cu") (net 6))
 (segment (start 130.774999 94.19) (end 129.8 94.19) (width 0.2) (layer "F.Cu") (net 6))
 (segment (start 107.75 112.25) (end 107.75 108.65) (width 0.2) (layer "F.Cu") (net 6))
 (segment (start 104 112.5) (end 107.5 112.5) (width 0.2) (layer "F.Cu") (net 6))
 (segment (start 91.810987 82.078) (end 88.839 85.049987) (width 0.2) (layer "F.Cu") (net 6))
 (segment (start 88.839 97.339) (end 104 112.5) (width 0.2) (layer "F.Cu") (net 6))
 (segment (start 126.126 96.389032) (end 125.865968 96.129) (width 0.2) (layer "F.Cu") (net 6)))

